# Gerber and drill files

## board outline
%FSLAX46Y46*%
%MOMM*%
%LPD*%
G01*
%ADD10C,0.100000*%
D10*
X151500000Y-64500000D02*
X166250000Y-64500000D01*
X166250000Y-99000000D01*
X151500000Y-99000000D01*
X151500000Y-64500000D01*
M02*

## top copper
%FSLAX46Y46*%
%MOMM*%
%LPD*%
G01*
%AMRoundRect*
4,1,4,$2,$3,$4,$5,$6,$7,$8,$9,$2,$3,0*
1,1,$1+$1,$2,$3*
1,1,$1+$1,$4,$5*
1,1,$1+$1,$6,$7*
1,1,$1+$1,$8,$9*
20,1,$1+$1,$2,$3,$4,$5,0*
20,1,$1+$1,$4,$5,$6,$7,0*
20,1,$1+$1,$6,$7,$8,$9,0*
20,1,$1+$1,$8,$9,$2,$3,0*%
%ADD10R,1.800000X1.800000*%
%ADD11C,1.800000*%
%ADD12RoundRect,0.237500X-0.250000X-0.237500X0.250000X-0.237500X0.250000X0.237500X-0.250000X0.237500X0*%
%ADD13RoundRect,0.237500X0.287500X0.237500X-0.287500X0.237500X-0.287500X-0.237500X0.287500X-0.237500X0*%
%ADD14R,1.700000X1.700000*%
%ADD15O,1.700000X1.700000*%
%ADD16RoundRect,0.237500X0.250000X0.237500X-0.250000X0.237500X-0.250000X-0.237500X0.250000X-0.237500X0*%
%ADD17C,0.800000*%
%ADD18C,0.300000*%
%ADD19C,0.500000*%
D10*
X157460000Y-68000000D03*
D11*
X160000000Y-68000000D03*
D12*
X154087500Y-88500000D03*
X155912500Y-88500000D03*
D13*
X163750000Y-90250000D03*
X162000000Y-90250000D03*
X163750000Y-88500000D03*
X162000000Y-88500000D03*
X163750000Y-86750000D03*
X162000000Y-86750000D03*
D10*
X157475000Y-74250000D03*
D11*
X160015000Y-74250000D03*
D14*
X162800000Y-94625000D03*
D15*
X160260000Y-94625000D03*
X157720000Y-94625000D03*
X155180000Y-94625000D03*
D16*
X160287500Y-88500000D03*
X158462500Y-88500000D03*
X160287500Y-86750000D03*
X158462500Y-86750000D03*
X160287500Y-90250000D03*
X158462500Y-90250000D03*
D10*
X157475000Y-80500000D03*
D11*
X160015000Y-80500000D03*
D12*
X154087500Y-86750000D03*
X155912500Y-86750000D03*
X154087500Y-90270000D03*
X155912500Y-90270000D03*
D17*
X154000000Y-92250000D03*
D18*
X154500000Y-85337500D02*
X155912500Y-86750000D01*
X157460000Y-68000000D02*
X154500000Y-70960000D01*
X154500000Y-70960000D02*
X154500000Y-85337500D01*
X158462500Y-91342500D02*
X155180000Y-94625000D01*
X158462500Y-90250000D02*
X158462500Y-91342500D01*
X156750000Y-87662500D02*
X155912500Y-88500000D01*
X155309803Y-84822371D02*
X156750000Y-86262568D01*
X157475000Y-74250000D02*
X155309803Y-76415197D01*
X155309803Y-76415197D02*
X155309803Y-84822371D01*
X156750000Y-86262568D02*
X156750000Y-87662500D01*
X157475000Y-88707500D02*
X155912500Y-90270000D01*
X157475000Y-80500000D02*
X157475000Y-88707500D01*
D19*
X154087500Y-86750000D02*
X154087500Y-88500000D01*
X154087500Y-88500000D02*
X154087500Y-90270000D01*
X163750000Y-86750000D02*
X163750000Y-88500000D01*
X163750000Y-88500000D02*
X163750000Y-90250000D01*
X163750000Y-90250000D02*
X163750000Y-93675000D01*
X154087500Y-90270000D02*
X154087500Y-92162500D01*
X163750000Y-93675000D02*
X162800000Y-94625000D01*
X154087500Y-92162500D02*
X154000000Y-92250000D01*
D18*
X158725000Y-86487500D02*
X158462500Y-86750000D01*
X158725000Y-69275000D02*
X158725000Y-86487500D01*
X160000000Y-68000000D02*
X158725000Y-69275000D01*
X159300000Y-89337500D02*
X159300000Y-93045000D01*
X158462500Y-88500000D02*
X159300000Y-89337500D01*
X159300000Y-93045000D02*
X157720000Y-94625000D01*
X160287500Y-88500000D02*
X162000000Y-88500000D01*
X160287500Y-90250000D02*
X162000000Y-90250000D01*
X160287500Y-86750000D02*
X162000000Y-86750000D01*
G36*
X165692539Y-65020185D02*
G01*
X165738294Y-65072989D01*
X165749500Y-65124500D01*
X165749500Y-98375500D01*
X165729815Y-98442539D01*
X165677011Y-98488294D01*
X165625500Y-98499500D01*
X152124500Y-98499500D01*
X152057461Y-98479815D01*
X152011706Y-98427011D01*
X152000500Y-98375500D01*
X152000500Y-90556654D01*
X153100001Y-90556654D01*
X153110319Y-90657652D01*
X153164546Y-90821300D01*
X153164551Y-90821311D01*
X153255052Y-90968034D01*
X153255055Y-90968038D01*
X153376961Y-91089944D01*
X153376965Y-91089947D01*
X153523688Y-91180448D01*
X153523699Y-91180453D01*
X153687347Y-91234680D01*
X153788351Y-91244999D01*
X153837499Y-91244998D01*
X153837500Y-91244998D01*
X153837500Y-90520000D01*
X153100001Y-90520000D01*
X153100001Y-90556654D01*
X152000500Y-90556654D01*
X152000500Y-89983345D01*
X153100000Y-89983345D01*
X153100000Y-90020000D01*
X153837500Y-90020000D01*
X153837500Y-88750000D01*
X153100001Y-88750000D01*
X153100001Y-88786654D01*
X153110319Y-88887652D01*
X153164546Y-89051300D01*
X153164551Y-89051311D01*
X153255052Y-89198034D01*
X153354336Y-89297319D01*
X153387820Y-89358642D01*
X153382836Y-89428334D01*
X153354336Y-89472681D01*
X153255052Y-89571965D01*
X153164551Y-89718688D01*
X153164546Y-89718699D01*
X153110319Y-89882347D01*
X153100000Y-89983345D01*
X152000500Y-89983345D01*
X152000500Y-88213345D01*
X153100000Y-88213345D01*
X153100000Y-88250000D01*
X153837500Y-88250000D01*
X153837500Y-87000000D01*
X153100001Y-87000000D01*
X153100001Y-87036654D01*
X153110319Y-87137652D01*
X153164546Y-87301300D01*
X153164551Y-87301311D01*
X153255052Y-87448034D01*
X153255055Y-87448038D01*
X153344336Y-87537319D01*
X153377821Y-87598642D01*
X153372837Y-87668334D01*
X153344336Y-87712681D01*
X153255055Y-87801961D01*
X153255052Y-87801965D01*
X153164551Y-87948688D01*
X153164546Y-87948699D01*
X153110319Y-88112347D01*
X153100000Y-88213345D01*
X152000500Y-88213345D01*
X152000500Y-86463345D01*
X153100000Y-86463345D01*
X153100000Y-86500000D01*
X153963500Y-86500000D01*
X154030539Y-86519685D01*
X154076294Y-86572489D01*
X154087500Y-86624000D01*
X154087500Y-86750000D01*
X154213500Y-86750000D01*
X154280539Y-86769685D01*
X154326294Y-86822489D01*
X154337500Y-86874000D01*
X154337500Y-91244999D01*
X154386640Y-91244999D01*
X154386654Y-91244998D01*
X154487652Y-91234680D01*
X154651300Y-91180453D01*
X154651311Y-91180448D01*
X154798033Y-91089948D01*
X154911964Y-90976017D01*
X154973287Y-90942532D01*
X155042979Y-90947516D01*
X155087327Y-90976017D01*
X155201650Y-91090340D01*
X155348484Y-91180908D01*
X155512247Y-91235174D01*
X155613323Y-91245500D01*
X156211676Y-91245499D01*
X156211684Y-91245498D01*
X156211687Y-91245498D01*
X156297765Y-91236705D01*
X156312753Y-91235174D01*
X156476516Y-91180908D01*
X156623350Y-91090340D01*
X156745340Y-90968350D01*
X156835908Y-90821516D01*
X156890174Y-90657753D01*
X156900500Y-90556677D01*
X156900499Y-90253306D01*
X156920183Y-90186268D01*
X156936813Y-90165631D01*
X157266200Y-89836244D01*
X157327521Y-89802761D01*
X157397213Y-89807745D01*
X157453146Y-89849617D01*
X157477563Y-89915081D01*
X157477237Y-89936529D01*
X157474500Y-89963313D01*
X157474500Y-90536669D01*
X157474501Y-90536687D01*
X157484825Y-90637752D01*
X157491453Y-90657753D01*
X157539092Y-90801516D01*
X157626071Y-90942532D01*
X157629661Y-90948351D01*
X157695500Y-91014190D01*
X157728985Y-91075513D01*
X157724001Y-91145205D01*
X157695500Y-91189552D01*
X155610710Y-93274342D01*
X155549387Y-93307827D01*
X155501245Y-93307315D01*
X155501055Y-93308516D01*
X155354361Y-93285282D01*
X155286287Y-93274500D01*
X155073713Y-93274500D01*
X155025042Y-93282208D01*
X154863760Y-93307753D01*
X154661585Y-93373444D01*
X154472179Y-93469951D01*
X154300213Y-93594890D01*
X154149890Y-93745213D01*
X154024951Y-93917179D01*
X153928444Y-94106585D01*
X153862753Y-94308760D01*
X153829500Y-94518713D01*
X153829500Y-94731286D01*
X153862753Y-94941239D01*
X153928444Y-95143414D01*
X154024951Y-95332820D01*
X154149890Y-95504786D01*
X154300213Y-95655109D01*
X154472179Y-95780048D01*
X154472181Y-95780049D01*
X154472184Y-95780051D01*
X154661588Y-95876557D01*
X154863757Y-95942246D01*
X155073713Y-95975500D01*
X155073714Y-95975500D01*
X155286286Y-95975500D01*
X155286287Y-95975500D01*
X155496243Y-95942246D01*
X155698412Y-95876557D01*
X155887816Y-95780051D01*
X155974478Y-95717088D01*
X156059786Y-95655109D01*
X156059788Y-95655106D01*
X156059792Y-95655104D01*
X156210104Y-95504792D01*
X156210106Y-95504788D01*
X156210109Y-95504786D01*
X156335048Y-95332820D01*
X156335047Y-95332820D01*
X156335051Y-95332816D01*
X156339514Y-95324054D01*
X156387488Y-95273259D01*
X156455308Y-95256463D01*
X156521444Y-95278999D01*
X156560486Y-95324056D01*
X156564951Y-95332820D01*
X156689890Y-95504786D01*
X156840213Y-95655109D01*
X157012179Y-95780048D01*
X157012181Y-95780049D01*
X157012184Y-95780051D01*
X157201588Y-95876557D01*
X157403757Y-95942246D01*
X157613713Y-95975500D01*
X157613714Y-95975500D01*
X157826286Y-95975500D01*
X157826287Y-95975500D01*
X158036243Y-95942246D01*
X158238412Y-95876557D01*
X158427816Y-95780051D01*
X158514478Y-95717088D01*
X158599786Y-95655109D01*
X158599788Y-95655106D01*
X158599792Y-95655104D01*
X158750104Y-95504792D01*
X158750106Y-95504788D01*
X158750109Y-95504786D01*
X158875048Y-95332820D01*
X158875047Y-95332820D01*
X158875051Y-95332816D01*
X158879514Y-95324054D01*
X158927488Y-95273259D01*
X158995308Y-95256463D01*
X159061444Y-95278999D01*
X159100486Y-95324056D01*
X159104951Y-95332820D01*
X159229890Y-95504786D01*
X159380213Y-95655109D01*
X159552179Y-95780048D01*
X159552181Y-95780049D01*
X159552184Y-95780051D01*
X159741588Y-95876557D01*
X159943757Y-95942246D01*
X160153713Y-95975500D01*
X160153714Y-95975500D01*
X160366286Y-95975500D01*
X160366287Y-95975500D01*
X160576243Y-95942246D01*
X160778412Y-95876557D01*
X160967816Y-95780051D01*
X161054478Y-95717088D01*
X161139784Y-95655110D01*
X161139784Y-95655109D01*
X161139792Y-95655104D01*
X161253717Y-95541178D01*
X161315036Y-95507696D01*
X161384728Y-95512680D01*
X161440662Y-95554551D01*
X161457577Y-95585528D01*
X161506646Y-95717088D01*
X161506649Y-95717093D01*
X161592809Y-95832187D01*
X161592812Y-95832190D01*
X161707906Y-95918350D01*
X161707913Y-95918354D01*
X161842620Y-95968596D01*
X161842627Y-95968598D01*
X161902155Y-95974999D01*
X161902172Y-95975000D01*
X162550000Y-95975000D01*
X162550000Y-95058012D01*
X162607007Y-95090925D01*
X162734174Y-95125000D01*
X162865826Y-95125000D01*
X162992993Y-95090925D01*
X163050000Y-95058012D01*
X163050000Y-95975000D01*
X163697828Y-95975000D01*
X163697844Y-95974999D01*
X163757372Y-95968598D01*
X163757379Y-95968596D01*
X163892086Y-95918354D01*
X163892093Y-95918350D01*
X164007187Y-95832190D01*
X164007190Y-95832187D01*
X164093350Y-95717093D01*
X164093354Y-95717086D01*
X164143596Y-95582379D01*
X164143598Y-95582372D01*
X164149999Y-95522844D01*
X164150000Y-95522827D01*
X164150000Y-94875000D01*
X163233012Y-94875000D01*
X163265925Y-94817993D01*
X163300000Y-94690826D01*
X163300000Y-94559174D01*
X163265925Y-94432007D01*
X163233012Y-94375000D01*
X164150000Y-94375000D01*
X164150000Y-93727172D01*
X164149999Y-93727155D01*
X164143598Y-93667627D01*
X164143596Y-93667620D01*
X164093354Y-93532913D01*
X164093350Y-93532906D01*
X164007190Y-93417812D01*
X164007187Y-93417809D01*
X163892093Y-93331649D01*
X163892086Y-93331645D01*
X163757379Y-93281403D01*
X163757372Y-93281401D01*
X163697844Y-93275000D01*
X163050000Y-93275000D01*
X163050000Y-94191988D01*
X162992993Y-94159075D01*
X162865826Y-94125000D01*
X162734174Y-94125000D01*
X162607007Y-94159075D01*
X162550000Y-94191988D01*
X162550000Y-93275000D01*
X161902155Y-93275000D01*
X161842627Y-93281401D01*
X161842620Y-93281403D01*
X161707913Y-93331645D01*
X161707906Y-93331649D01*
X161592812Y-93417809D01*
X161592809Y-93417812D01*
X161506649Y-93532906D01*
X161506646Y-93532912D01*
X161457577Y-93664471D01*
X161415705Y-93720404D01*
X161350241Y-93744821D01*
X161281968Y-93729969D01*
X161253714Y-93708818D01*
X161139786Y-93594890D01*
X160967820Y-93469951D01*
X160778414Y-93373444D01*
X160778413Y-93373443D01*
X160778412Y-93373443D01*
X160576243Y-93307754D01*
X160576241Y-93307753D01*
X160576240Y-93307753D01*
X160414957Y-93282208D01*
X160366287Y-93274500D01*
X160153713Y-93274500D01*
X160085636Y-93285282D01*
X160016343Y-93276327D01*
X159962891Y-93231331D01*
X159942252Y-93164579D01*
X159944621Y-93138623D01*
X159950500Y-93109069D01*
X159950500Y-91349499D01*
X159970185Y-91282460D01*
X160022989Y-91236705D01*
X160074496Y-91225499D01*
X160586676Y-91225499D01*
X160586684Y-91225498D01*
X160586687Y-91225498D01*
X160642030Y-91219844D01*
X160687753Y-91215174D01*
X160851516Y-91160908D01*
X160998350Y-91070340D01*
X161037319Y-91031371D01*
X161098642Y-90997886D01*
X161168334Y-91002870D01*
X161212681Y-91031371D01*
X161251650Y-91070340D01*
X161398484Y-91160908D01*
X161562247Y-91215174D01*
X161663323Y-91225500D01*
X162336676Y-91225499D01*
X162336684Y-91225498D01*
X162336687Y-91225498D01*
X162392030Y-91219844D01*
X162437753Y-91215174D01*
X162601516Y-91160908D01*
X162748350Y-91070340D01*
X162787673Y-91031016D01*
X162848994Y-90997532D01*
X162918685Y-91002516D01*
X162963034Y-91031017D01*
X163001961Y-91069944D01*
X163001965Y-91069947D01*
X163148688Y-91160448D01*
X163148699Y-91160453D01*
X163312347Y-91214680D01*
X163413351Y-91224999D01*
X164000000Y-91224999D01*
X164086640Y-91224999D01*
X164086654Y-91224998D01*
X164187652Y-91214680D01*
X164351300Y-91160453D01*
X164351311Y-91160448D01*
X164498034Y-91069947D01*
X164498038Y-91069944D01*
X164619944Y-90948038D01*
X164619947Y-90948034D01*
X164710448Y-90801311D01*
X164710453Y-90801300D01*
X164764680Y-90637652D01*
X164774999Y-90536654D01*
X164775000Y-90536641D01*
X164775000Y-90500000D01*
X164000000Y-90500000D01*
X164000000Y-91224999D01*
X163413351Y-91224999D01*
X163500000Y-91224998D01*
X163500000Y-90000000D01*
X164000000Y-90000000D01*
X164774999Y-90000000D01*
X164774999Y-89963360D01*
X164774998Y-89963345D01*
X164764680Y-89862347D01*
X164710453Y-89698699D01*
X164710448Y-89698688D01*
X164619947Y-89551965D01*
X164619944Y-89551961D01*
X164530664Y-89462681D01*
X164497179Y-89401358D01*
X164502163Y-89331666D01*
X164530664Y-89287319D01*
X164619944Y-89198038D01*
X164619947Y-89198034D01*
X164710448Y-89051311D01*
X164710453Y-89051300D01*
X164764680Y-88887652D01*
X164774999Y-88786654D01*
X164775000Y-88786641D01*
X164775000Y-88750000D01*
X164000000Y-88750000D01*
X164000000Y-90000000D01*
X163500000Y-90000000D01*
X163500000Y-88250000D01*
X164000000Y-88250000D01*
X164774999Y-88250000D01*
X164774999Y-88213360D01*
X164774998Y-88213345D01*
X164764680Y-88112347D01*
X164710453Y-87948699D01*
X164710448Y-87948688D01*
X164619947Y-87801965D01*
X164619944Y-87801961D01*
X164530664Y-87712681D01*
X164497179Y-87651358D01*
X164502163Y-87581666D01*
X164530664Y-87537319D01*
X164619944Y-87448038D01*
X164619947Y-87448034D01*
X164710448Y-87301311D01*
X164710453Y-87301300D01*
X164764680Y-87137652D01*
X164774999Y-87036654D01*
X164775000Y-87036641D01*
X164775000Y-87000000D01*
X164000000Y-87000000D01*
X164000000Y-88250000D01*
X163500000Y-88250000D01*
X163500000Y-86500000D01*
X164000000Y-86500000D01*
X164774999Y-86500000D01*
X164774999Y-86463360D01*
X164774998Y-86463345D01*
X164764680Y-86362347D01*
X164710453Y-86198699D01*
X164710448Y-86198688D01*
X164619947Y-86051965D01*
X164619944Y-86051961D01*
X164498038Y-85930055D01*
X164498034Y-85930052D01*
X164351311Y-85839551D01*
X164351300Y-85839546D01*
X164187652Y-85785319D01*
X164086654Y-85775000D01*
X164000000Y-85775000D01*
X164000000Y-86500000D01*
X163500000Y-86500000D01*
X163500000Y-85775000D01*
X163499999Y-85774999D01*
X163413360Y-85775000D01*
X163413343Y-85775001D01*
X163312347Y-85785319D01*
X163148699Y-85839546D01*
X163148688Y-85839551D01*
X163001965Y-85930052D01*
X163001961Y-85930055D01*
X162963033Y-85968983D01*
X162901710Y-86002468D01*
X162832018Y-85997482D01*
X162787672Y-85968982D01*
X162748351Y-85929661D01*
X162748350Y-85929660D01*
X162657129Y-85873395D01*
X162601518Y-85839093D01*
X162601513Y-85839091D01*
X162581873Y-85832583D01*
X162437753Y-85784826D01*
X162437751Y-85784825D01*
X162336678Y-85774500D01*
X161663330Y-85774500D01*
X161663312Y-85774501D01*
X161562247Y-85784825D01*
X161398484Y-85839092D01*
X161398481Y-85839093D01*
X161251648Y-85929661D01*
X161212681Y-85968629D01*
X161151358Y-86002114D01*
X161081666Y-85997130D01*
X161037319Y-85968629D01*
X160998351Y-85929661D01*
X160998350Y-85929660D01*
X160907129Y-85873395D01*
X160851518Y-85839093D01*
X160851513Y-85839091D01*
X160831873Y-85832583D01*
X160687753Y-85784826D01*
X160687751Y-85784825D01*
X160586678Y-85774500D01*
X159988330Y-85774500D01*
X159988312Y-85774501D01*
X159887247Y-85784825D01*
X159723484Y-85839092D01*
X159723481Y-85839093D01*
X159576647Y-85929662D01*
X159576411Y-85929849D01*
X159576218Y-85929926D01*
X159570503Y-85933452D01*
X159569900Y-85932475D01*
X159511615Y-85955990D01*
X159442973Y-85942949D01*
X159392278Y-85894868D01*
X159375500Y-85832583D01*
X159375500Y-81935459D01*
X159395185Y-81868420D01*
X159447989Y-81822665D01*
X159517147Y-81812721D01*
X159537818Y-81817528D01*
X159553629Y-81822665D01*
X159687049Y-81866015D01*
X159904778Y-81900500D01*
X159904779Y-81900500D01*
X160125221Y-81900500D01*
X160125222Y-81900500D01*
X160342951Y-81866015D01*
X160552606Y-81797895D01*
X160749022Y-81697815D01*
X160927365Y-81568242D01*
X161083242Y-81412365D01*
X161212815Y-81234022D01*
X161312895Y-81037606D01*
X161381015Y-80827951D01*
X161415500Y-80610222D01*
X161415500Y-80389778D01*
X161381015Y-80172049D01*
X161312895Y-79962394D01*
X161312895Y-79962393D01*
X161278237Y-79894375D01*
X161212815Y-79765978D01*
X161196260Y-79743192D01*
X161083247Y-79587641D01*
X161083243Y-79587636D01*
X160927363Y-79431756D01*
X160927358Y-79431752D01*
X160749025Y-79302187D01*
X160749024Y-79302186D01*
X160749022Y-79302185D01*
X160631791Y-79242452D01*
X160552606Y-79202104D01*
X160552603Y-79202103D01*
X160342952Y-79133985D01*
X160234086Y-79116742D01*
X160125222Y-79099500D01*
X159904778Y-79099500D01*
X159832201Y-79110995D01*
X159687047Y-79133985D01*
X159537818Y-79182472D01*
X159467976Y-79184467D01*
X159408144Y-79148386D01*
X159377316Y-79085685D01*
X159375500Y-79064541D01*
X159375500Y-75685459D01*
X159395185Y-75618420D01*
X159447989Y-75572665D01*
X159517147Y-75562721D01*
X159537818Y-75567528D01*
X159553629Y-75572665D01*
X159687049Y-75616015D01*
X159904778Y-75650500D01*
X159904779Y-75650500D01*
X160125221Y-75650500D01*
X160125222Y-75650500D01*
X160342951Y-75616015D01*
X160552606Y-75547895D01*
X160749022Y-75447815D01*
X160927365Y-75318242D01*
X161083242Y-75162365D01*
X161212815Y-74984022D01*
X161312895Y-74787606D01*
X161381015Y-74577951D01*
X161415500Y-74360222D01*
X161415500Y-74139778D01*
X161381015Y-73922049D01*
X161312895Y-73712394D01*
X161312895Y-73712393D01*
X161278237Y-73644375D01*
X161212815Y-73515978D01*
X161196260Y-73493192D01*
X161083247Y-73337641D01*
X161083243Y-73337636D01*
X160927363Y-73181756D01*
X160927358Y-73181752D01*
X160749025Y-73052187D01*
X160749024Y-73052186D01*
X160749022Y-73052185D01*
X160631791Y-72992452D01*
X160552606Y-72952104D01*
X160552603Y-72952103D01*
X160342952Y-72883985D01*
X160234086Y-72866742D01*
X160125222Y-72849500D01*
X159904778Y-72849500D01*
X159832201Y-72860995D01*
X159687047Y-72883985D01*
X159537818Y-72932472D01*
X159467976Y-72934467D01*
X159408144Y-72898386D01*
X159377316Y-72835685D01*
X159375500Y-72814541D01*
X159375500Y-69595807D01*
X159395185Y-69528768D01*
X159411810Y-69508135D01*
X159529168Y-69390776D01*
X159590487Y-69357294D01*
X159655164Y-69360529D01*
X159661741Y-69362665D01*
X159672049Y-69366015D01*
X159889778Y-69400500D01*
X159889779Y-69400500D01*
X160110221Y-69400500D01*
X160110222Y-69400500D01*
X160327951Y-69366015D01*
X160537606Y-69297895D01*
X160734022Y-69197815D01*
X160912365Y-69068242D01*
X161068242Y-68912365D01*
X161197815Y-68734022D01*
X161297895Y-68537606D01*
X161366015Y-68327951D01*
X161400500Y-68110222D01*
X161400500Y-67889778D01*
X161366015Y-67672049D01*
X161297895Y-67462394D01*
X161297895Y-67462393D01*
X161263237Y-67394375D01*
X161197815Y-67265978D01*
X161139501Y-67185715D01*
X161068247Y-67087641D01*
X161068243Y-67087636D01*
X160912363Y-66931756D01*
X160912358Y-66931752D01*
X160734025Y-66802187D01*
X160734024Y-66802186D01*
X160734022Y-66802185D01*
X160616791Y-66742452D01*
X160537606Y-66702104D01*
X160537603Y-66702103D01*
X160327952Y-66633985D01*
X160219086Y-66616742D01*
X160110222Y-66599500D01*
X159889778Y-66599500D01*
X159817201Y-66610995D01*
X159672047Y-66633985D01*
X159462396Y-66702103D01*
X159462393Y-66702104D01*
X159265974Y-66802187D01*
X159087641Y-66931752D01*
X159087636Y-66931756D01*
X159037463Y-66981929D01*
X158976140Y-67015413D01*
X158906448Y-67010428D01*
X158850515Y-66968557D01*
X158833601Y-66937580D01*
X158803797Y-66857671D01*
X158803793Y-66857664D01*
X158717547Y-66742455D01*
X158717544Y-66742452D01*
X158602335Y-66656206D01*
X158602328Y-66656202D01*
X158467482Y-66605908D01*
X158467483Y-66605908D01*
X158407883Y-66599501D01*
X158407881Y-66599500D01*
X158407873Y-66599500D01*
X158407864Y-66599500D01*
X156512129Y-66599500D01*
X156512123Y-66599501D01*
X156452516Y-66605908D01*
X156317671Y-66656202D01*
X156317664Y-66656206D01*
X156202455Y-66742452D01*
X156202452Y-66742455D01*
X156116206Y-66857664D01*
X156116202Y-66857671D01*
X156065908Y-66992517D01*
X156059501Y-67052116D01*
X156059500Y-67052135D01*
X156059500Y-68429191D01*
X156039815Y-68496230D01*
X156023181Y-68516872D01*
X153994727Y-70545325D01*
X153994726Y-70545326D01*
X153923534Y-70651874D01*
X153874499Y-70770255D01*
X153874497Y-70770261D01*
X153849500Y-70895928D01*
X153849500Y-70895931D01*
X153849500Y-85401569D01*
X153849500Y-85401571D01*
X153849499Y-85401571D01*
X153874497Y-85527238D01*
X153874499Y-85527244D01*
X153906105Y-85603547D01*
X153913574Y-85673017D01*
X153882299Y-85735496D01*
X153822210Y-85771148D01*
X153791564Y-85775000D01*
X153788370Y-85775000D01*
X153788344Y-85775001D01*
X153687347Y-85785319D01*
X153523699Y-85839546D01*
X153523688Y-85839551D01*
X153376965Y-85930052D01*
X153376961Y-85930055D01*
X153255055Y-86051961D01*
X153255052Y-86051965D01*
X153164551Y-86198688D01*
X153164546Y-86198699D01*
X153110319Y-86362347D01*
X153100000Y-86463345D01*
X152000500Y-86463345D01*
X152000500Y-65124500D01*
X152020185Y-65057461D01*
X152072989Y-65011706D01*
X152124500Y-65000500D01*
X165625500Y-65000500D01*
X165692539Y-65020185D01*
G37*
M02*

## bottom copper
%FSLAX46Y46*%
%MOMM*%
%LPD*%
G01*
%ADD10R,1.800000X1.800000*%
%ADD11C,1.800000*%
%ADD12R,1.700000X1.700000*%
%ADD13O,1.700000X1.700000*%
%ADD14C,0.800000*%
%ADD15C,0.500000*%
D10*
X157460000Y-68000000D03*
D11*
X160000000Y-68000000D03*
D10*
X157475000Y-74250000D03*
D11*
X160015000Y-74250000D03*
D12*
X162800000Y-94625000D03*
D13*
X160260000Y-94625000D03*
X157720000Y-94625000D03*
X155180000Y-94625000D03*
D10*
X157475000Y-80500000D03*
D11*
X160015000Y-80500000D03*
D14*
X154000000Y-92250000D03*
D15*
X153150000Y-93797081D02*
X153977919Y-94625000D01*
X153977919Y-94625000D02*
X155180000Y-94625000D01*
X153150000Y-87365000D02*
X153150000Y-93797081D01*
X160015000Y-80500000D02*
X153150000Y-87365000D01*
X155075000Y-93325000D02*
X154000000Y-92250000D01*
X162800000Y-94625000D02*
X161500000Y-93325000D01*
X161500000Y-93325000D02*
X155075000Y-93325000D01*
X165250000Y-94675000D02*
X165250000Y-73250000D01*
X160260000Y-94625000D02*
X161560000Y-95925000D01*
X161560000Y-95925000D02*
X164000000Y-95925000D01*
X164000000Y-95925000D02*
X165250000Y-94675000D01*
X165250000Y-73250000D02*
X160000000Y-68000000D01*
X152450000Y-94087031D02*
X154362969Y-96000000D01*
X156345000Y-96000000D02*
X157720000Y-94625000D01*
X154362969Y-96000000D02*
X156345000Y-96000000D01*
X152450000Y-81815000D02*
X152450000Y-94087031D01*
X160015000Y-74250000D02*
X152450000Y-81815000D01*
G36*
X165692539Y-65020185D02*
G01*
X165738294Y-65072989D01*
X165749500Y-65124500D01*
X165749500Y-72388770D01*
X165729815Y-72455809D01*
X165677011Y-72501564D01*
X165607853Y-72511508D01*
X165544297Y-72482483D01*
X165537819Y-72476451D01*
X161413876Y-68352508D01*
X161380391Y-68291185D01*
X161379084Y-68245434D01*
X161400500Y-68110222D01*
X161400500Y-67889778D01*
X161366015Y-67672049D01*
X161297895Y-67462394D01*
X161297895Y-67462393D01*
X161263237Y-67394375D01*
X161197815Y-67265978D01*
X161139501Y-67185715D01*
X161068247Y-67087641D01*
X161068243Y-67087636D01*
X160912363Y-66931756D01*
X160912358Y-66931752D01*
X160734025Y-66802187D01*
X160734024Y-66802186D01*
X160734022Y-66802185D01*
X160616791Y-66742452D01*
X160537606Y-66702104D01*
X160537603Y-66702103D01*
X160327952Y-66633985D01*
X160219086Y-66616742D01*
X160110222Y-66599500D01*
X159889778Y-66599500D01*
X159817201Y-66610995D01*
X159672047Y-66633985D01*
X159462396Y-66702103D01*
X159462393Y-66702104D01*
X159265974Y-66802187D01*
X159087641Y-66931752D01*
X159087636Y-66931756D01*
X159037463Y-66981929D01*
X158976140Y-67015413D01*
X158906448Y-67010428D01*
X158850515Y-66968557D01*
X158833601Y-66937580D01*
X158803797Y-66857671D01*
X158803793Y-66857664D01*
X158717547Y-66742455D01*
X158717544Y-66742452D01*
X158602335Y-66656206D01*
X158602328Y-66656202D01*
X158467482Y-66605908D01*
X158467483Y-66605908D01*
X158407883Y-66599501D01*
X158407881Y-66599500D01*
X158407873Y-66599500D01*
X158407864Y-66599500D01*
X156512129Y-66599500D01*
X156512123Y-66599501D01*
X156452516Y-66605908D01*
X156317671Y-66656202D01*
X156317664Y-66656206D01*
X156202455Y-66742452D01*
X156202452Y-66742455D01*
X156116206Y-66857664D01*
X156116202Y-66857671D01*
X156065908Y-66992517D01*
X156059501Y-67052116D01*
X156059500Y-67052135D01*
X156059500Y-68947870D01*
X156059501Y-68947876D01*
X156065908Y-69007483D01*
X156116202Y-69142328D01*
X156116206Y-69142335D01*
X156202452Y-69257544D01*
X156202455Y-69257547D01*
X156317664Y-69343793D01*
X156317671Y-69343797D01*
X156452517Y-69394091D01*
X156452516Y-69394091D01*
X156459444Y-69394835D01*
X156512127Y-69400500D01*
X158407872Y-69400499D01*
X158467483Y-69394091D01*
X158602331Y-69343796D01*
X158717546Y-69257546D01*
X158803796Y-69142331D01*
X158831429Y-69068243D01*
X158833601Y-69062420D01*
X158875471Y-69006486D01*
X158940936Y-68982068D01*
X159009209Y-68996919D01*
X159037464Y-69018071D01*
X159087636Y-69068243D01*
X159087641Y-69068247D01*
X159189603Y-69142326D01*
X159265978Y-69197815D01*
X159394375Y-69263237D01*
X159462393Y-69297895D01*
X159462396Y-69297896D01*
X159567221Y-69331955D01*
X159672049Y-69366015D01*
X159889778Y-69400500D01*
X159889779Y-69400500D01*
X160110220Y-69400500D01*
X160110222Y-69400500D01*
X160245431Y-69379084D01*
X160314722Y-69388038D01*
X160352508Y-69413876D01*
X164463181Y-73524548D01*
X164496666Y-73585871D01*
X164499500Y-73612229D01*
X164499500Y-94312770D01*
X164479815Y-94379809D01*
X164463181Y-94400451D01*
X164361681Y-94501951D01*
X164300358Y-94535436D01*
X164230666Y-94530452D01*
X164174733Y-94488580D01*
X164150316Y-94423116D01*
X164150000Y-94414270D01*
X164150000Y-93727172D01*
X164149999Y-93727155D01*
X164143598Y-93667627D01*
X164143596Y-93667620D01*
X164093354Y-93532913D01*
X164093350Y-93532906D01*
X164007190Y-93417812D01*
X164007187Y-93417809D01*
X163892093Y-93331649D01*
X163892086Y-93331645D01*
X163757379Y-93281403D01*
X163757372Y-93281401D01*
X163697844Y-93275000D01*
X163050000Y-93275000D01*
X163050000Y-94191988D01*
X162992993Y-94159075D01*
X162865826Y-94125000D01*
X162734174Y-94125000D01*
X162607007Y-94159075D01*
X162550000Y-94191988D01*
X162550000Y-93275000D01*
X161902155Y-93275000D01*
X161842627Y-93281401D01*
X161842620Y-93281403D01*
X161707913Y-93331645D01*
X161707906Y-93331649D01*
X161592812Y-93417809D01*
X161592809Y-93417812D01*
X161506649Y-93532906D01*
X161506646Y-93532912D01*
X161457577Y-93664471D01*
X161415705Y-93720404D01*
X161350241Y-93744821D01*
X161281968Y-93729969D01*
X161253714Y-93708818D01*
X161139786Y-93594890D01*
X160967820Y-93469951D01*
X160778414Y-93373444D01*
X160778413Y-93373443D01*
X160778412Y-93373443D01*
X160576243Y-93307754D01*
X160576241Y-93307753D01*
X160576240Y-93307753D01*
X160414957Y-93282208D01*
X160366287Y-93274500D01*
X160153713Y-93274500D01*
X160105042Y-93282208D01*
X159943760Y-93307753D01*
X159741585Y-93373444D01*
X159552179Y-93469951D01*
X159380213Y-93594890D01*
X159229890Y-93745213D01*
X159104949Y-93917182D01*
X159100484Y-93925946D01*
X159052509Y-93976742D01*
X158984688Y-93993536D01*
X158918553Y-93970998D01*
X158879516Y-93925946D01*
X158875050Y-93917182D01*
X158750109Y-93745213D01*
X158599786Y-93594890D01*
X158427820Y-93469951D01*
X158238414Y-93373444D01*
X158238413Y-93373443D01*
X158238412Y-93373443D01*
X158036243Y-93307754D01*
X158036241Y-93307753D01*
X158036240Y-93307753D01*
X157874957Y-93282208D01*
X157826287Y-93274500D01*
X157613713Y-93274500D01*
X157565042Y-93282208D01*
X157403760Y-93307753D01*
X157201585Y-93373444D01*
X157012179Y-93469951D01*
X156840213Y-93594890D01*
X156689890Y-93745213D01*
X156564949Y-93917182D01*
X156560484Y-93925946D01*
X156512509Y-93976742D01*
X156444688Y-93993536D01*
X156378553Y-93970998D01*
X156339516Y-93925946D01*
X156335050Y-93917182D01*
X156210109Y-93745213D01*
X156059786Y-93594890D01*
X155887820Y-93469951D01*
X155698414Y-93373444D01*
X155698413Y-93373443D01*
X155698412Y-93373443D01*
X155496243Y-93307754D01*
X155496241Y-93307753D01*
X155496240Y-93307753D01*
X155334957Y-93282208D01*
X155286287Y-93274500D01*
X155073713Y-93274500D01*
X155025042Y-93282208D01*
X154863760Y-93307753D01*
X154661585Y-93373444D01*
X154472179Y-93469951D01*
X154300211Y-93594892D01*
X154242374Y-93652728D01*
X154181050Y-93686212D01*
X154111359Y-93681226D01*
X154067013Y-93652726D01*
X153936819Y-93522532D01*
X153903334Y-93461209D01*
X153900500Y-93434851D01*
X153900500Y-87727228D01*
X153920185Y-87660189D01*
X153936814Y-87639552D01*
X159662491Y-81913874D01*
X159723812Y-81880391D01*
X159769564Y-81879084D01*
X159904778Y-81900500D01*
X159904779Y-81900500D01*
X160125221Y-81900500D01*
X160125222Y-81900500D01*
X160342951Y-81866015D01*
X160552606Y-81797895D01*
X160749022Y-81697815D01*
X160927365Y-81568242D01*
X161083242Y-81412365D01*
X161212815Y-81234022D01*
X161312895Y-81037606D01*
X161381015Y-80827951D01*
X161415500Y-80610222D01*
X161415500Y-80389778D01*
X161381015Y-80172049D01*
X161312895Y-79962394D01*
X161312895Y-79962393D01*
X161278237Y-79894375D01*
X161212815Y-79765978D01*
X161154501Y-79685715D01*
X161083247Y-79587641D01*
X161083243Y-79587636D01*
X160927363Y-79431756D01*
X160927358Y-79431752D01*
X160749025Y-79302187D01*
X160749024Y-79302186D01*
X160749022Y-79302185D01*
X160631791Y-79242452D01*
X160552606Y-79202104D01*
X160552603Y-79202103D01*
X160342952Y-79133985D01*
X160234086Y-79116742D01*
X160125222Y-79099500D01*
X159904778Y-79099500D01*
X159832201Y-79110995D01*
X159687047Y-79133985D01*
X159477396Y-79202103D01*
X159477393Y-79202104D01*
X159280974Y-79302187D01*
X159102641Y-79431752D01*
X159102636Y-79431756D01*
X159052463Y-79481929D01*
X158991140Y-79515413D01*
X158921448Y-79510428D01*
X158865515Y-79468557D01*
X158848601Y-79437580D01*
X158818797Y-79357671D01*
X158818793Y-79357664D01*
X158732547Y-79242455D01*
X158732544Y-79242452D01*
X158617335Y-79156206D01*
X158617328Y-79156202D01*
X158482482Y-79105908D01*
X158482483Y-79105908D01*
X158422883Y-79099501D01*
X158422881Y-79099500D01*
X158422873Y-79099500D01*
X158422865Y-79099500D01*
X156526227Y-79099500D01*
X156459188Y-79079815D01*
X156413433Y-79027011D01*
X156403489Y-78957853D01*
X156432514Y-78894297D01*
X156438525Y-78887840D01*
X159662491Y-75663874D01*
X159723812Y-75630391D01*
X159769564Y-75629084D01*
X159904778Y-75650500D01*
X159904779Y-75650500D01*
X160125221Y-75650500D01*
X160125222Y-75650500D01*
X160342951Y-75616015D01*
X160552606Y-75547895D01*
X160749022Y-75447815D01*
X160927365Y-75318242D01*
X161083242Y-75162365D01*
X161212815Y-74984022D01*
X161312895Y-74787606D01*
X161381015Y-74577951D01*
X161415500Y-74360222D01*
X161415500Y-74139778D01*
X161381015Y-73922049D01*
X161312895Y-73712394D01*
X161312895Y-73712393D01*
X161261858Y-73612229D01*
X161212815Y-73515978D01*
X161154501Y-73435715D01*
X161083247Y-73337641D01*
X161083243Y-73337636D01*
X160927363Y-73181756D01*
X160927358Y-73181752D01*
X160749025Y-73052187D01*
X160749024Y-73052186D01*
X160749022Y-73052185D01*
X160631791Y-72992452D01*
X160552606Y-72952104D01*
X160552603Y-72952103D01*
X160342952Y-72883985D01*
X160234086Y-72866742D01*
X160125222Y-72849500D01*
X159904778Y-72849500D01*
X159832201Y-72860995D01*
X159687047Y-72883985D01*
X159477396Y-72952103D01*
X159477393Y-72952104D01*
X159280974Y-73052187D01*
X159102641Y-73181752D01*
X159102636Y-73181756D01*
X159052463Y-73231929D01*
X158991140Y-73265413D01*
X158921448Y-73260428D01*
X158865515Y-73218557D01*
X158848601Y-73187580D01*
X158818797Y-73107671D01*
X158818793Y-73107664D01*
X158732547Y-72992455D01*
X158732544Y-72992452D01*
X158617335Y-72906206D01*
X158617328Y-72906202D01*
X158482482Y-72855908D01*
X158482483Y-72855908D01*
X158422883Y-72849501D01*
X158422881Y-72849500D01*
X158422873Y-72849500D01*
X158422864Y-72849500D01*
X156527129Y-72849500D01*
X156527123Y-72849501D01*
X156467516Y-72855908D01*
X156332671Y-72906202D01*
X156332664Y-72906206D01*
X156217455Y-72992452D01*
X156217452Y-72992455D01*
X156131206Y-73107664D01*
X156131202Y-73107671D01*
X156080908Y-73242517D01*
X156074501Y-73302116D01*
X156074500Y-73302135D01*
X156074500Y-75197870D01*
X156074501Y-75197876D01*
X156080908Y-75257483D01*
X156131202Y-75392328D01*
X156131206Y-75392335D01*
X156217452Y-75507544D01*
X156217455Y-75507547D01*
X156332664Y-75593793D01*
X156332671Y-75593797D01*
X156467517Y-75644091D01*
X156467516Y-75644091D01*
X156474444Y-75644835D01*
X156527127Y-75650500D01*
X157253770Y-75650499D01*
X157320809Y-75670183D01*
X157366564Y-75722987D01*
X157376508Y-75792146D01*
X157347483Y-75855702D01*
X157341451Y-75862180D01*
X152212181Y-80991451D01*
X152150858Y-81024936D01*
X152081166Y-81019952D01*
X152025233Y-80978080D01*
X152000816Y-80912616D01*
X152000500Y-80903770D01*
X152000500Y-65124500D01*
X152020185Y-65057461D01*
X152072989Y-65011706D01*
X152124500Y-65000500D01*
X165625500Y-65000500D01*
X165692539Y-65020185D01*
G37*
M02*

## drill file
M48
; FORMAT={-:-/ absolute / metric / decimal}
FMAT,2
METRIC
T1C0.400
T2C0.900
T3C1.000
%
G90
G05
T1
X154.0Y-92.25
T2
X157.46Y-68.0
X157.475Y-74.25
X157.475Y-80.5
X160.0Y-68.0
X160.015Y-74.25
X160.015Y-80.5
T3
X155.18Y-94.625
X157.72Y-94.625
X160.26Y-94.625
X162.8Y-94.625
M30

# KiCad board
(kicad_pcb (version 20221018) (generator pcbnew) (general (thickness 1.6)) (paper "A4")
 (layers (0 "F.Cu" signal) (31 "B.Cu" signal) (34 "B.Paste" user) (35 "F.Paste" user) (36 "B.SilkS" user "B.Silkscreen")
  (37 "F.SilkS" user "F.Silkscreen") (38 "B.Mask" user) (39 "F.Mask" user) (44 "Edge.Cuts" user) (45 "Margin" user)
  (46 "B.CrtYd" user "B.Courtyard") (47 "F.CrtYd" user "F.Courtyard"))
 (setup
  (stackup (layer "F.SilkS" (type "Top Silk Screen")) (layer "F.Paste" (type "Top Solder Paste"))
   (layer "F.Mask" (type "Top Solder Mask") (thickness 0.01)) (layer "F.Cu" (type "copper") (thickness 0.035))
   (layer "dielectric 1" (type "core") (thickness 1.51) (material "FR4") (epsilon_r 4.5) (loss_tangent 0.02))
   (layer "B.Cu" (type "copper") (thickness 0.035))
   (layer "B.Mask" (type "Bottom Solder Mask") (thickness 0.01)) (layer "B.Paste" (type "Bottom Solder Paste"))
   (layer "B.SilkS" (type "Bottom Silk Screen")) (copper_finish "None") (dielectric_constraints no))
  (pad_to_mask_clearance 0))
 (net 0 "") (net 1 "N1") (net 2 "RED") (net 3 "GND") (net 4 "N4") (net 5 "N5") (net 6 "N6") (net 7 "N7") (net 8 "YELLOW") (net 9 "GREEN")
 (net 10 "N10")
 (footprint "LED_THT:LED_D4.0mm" (layer "F.Cu") (at 157.46 68)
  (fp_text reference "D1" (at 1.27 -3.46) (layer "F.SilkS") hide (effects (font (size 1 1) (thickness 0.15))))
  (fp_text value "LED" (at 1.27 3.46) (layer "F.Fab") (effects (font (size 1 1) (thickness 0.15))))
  (pad "1" thru_hole rect (at 0 0) (size 1.8 1.8) (drill 0.9) (layers "*.Cu" "*.Mask") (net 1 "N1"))
  (pad "2" thru_hole circle (at 2.54 0) (size 1.8 1.8) (drill 0.9) (layers "*.Cu" "*.Mask") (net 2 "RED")))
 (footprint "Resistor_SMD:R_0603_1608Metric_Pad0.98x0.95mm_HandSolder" (layer "F.Cu") (at 155 88.5)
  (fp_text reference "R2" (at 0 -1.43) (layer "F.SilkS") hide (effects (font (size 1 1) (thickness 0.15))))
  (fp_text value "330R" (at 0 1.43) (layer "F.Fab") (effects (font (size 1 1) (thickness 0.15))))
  (pad "1" smd roundrect (at -0.9125 0) (size 0.975 0.95) (layers "F.Cu" "F.Paste" "F.Mask") (roundrect_rratio 0.25) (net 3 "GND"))
  (pad "2" smd roundrect (at 0.9125 0) (size 0.975 0.95) (layers "F.Cu" "F.Paste" "F.Mask") (roundrect_rratio 0.25) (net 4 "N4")))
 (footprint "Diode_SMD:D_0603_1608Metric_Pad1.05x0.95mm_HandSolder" (layer "F.Cu") (at 162.875 90.25 180)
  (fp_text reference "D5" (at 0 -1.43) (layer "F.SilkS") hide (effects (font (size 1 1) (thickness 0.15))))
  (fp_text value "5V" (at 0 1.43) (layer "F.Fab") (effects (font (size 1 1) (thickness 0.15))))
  (pad "1" smd roundrect (at -0.875 0 180) (size 1.05 0.95) (layers "F.Cu" "F.Paste" "F.Mask") (roundrect_rratio 0.25) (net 3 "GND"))
  (pad "2" smd roundrect (at 0.875 0 180) (size 1.05 0.95) (layers "F.Cu" "F.Paste" "F.Mask") (roundrect_rratio 0.25) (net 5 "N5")))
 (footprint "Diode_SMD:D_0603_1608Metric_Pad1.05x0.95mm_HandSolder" (layer "F.Cu") (at 162.875 88.5 180)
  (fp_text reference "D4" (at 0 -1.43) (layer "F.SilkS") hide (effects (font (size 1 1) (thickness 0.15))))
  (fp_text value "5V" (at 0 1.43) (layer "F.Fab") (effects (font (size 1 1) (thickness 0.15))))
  (pad "1" smd roundrect (at -0.875 0 180) (size 1.05 0.95) (layers "F.Cu" "F.Paste" "F.Mask") (roundrect_rratio 0.25) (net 3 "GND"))
  (pad "2" smd roundrect (at 0.875 0 180) (size 1.05 0.95) (layers "F.Cu" "F.Paste" "F.Mask") (roundrect_rratio 0.25) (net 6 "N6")))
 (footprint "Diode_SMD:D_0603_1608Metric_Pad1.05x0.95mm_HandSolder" (layer "F.Cu") (at 162.875 86.75 180)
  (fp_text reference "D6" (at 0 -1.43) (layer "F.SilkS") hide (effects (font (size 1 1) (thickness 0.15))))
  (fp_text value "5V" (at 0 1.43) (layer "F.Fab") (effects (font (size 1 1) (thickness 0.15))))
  (pad "1" smd roundrect (at -0.875 0 180) (size 1.05 0.95) (layers "F.Cu" "F.Paste" "F.Mask") (roundrect_rratio 0.25) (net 3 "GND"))
  (pad "2" smd roundrect (at 0.875 0 180) (size 1.05 0.95) (layers "F.Cu" "F.Paste" "F.Mask") (roundrect_rratio 0.25) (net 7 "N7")))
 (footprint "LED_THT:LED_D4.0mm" (layer "F.Cu") (at 157.475 74.25)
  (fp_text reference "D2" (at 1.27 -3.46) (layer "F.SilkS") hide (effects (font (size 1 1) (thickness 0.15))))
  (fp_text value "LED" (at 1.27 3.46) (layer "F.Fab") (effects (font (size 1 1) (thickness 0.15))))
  (pad "1" thru_hole rect (at 0 0) (size 1.8 1.8) (drill 0.9) (layers "*.Cu" "*.Mask") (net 4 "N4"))
  (pad "2" thru_hole circle (at 2.54 0) (size 1.8 1.8) (drill 0.9) (layers "*.Cu" "*.Mask") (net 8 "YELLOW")))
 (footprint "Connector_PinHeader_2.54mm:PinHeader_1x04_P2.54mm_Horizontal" (layer "F.Cu") (at 162.8 94.625 -90)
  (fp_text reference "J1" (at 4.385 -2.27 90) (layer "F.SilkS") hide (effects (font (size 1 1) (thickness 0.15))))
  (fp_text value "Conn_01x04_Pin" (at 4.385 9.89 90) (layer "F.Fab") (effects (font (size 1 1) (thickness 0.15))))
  (pad "1" thru_hole rect (at 0 0 270) (size 1.7 1.7) (drill 1) (layers "*.Cu" "*.Mask") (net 3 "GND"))
  (pad "2" thru_hole oval (at 0 2.54 270) (size 1.7 1.7) (drill 1) (layers "*.Cu" "*.Mask") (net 2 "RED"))
  (pad "3" thru_hole oval (at 0 5.08 270) (size 1.7 1.7) (drill 1) (layers "*.Cu" "*.Mask") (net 8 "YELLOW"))
  (pad "4" thru_hole oval (at 0 7.62 270) (size 1.7 1.7) (drill 1) (layers "*.Cu" "*.Mask") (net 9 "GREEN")))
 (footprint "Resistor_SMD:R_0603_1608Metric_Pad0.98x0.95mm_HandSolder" (layer "F.Cu") (at 159.375 88.5 180)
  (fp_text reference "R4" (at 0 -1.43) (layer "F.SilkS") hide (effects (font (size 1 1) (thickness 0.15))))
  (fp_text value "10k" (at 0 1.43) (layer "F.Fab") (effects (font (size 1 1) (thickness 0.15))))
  (pad "1" smd roundrect (at -0.9125 0 180) (size 0.975 0.95) (layers "F.Cu" "F.Paste" "F.Mask") (roundrect_rratio 0.25) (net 6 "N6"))
  (pad "2" smd roundrect (at 0.9125 0 180) (size 0.975 0.95) (layers "F.Cu" "F.Paste" "F.Mask") (roundrect_rratio 0.25) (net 8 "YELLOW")))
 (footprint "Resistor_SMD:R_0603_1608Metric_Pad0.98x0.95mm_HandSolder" (layer "F.Cu") (at 159.375 86.75 180)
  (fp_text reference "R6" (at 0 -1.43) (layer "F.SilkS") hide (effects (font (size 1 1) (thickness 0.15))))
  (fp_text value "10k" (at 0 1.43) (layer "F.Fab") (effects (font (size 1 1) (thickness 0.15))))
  (pad "1" smd roundrect (at -0.9125 0 180) (size 0.975 0.95) (layers "F.Cu" "F.Paste" "F.Mask") (roundrect_rratio 0.25) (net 7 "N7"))
  (pad "2" smd roundrect (at 0.9125 0 180) (size 0.975 0.95) (layers "F.Cu" "F.Paste" "F.Mask") (roundrect_rratio 0.25) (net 2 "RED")))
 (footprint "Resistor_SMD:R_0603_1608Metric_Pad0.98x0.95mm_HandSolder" (layer "F.Cu") (at 159.375 90.25 180)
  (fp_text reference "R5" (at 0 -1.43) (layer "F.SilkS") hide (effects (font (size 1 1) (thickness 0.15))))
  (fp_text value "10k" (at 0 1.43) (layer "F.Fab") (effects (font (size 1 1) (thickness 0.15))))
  (pad "1" smd roundrect (at -0.9125 0 180) (size 0.975 0.95) (layers "F.Cu" "F.Paste" "F.Mask") (roundrect_rratio 0.25) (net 5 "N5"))
  (pad "2" smd roundrect (at 0.9125 0 180) (size 0.975 0.95) (layers "F.Cu" "F.Paste" "F.Mask") (roundrect_rratio 0.25) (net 9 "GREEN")))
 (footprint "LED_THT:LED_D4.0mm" (layer "F.Cu") (at 157.475 80.5)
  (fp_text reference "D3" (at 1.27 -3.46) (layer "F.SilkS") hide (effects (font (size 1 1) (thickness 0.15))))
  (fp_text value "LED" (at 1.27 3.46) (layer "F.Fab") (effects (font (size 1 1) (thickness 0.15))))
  (pad "1" thru_hole rect (at 0 0) (size 1.8 1.8) (drill 0.9) (layers "*.Cu" "*.Mask") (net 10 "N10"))
  (pad "2" thru_hole circle (at 2.54 0) (size 1.8 1.8) (drill 0.9) (layers "*.Cu" "*.Mask") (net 9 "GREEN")))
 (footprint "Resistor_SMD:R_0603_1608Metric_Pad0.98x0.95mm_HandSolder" (layer "F.Cu") (at 155 86.75)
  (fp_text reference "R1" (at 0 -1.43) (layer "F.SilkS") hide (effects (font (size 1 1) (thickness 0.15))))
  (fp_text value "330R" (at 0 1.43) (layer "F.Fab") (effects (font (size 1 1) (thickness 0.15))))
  (pad "1" smd roundrect (at -0.9125 0) (size 0.975 0.95) (layers "F.Cu" "F.Paste" "F.Mask") (roundrect_rratio 0.25) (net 3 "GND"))
  (pad "2" smd roundrect (at 0.9125 0) (size 0.975 0.95) (layers "F.Cu" "F.Paste" "F.Mask") (roundrect_rratio 0.25) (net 1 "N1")))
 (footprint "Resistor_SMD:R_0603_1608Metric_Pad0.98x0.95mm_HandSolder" (layer "F.Cu") (at 155 90.27)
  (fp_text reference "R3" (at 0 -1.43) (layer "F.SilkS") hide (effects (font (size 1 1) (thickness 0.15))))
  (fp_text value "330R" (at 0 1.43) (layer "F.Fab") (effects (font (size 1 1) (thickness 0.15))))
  (pad "1" smd roundrect (at -0.9125 0) (size 0.975 0.95) (layers "F.Cu" "F.Paste" "F.Mask") (roundrect_rratio 0.25) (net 3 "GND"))
  (pad "2" smd roundrect (at 0.9125 0) (size 0.975 0.95) (layers "F.Cu" "F.Paste" "F.Mask") (roundrect_rratio 0.25) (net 10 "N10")))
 (gr_rect (start 151.5 64.5) (end 166.25 99) (stroke (width 0.1) (type default)) (fill none) (layer "Edge.Cuts"))
 (segment (start 154.5 85.3375) (end 155.9125 86.75) (width 0.3) (layer "F.Cu") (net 1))
 (segment (start 157.46 68) (end 154.5 70.96) (width 0.3) (layer "F.Cu") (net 1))
 (segment (start 154.5 70.96) (end 154.5 85.3375) (width 0.3) (layer "F.Cu") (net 1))
 (segment (start 158.4625 91.3425) (end 155.18 94.625) (width 0.3) (layer "F.Cu") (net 9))
 (segment (start 158.4625 90.25) (end 158.4625 91.3425) (width 0.3) (layer "F.Cu") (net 9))
 (segment (start 153.15 93.797081) (end 153.977919 94.625) (width 0.5) (layer "B.Cu") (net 9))
 (segment (start 153.977919 94.625) (end 155.18 94.625) (width 0.5) (layer "B.Cu") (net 9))
 (segment (start 153.15 87.365) (end 153.15 93.797081) (width 0.5) (layer "B.Cu") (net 9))
 (segment (start 160.015 80.5) (end 153.15 87.365) (width 0.5) (layer "B.Cu") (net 9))
 (segment (start 156.75 87.6625) (end 155.9125 88.5) (width 0.3) (layer "F.Cu") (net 4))
 (segment (start 155.309803 84.822371) (end 156.75 86.262568) (width 0.3) (layer "F.Cu") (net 4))
 (segment (start 157.475 74.25) (end 155.309803 76.415197) (width 0.3) (layer "F.Cu") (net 4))
 (segment (start 155.309803 76.415197) (end 155.309803 84.822371) (width 0.3) (layer "F.Cu") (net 4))
 (segment (start 156.75 86.262568) (end 156.75 87.6625) (width 0.3) (layer "F.Cu") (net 4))
 (segment (start 157.475 88.7075) (end 155.9125 90.27) (width 0.3) (layer "F.Cu") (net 10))
 (segment (start 157.475 80.5) (end 157.475 88.7075) (width 0.3) (layer "F.Cu") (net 10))
 (segment (start 154.0875 86.75) (end 154.0875 88.5) (width 0.5) (layer "F.Cu") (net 3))
 (segment (start 154.0875 88.5) (end 154.0875 90.27) (width 0.5) (layer "F.Cu") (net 3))
 (segment (start 163.75 86.75) (end 163.75 88.5) (width 0.5) (layer "F.Cu") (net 3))
 (segment (start 163.75 88.5) (end 163.75 90.25) (width 0.5) (layer "F.Cu") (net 3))
 (segment (start 163.75 90.25) (end 163.75 93.675) (width 0.5) (layer "F.Cu") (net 3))
 (segment (start 154.0875 90.27) (end 154.0875 92.1625) (width 0.5) (layer "F.Cu") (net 3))
 (segment (start 163.75 93.675) (end 162.8 94.625) (width 0.5) (layer "F.Cu") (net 3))
 (segment (start 154.0875 92.1625) (end 154 92.25) (width 0.5) (layer "F.Cu") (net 3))
 (via (at 154 92.25) (size 0.8) (drill 0.4) (layers "F.Cu" "B.Cu") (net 3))
 (segment (start 155.075 93.325) (end 154 92.25) (width 0.5) (layer "B.Cu") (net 3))
 (segment (start 162.8 94.625) (end 161.5 93.325) (width 0.5) (layer "B.Cu") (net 3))
 (segment (start 161.5 93.325) (end 155.075 93.325) (width 0.5) (layer "B.Cu") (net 3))
 (segment (start 158.725 86.4875) (end 158.4625 86.75) (width 0.3) (layer "F.Cu") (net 2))
 (segment (start 158.725 69.275) (end 158.725 86.4875) (width 0.3) (layer "F.Cu") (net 2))
 (segment (start 160 68) (end 158.725 69.275) (width 0.3) (layer "F.Cu") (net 2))
 (segment (start 165.25 94.675) (end 165.25 73.25) (width 0.5) (layer "B.Cu") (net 2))
 (segment (start 160.26 94.625) (end 161.56 95.925) (width 0.5) (layer "B.Cu") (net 2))
 (segment (start 161.56 95.925) (end 164 95.925) (width 0.5) (layer "B.Cu") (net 2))
 (segment (start 164 95.925) (end 165.25 94.675) (width 0.5) (layer "B.Cu") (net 2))
 (segment (start 165.25 73.25) (end 160 68) (width 0.5) (layer "B.Cu") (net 2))
 (segment (start 159.3 89.3375) (end 159.3 93.045) (width 0.3) (layer "F.Cu") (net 8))
 (segment (start 158.4625 88.5) (end 159.3 89.3375) (width 0.3) (layer "F.Cu") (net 8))
 (segment (start 159.3 93.045) (end 157.72 94.625) (width 0.3) (layer "F.Cu") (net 8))
 (segment (start 152.45 94.087031) (end 154.362969 96) (width 0.5) (layer "B.Cu") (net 8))
 (segment (start 156.345 96) (end 157.72 94.625) (width 0.5) (layer "B.Cu") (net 8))
 (segment (start 154.362969 96) (end 156.345 96) (width 0.5) (layer "B.Cu") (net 8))
 (segment (start 152.45 81.815) (end 152.45 94.087031) (width 0.5) (layer "B.Cu") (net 8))
 (segment (start 160.015 74.25) (end 152.45 81.815) (width 0.5) (layer "B.Cu") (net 8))
 (segment (start 160.2875 88.5) (end 162 88.5) (width 0.3) (layer "F.Cu") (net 6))
 (segment (start 160.2875 90.25) (end 162 90.25) (width 0.3) (layer "F.Cu") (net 5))
 (segment (start 160.2875 86.75) (end 162 86.75) (width 0.3) (layer "F.Cu") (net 7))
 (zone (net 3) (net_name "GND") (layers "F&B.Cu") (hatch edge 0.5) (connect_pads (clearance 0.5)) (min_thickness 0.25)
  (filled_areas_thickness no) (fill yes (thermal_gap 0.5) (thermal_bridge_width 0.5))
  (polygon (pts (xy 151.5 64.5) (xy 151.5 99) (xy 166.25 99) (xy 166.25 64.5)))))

